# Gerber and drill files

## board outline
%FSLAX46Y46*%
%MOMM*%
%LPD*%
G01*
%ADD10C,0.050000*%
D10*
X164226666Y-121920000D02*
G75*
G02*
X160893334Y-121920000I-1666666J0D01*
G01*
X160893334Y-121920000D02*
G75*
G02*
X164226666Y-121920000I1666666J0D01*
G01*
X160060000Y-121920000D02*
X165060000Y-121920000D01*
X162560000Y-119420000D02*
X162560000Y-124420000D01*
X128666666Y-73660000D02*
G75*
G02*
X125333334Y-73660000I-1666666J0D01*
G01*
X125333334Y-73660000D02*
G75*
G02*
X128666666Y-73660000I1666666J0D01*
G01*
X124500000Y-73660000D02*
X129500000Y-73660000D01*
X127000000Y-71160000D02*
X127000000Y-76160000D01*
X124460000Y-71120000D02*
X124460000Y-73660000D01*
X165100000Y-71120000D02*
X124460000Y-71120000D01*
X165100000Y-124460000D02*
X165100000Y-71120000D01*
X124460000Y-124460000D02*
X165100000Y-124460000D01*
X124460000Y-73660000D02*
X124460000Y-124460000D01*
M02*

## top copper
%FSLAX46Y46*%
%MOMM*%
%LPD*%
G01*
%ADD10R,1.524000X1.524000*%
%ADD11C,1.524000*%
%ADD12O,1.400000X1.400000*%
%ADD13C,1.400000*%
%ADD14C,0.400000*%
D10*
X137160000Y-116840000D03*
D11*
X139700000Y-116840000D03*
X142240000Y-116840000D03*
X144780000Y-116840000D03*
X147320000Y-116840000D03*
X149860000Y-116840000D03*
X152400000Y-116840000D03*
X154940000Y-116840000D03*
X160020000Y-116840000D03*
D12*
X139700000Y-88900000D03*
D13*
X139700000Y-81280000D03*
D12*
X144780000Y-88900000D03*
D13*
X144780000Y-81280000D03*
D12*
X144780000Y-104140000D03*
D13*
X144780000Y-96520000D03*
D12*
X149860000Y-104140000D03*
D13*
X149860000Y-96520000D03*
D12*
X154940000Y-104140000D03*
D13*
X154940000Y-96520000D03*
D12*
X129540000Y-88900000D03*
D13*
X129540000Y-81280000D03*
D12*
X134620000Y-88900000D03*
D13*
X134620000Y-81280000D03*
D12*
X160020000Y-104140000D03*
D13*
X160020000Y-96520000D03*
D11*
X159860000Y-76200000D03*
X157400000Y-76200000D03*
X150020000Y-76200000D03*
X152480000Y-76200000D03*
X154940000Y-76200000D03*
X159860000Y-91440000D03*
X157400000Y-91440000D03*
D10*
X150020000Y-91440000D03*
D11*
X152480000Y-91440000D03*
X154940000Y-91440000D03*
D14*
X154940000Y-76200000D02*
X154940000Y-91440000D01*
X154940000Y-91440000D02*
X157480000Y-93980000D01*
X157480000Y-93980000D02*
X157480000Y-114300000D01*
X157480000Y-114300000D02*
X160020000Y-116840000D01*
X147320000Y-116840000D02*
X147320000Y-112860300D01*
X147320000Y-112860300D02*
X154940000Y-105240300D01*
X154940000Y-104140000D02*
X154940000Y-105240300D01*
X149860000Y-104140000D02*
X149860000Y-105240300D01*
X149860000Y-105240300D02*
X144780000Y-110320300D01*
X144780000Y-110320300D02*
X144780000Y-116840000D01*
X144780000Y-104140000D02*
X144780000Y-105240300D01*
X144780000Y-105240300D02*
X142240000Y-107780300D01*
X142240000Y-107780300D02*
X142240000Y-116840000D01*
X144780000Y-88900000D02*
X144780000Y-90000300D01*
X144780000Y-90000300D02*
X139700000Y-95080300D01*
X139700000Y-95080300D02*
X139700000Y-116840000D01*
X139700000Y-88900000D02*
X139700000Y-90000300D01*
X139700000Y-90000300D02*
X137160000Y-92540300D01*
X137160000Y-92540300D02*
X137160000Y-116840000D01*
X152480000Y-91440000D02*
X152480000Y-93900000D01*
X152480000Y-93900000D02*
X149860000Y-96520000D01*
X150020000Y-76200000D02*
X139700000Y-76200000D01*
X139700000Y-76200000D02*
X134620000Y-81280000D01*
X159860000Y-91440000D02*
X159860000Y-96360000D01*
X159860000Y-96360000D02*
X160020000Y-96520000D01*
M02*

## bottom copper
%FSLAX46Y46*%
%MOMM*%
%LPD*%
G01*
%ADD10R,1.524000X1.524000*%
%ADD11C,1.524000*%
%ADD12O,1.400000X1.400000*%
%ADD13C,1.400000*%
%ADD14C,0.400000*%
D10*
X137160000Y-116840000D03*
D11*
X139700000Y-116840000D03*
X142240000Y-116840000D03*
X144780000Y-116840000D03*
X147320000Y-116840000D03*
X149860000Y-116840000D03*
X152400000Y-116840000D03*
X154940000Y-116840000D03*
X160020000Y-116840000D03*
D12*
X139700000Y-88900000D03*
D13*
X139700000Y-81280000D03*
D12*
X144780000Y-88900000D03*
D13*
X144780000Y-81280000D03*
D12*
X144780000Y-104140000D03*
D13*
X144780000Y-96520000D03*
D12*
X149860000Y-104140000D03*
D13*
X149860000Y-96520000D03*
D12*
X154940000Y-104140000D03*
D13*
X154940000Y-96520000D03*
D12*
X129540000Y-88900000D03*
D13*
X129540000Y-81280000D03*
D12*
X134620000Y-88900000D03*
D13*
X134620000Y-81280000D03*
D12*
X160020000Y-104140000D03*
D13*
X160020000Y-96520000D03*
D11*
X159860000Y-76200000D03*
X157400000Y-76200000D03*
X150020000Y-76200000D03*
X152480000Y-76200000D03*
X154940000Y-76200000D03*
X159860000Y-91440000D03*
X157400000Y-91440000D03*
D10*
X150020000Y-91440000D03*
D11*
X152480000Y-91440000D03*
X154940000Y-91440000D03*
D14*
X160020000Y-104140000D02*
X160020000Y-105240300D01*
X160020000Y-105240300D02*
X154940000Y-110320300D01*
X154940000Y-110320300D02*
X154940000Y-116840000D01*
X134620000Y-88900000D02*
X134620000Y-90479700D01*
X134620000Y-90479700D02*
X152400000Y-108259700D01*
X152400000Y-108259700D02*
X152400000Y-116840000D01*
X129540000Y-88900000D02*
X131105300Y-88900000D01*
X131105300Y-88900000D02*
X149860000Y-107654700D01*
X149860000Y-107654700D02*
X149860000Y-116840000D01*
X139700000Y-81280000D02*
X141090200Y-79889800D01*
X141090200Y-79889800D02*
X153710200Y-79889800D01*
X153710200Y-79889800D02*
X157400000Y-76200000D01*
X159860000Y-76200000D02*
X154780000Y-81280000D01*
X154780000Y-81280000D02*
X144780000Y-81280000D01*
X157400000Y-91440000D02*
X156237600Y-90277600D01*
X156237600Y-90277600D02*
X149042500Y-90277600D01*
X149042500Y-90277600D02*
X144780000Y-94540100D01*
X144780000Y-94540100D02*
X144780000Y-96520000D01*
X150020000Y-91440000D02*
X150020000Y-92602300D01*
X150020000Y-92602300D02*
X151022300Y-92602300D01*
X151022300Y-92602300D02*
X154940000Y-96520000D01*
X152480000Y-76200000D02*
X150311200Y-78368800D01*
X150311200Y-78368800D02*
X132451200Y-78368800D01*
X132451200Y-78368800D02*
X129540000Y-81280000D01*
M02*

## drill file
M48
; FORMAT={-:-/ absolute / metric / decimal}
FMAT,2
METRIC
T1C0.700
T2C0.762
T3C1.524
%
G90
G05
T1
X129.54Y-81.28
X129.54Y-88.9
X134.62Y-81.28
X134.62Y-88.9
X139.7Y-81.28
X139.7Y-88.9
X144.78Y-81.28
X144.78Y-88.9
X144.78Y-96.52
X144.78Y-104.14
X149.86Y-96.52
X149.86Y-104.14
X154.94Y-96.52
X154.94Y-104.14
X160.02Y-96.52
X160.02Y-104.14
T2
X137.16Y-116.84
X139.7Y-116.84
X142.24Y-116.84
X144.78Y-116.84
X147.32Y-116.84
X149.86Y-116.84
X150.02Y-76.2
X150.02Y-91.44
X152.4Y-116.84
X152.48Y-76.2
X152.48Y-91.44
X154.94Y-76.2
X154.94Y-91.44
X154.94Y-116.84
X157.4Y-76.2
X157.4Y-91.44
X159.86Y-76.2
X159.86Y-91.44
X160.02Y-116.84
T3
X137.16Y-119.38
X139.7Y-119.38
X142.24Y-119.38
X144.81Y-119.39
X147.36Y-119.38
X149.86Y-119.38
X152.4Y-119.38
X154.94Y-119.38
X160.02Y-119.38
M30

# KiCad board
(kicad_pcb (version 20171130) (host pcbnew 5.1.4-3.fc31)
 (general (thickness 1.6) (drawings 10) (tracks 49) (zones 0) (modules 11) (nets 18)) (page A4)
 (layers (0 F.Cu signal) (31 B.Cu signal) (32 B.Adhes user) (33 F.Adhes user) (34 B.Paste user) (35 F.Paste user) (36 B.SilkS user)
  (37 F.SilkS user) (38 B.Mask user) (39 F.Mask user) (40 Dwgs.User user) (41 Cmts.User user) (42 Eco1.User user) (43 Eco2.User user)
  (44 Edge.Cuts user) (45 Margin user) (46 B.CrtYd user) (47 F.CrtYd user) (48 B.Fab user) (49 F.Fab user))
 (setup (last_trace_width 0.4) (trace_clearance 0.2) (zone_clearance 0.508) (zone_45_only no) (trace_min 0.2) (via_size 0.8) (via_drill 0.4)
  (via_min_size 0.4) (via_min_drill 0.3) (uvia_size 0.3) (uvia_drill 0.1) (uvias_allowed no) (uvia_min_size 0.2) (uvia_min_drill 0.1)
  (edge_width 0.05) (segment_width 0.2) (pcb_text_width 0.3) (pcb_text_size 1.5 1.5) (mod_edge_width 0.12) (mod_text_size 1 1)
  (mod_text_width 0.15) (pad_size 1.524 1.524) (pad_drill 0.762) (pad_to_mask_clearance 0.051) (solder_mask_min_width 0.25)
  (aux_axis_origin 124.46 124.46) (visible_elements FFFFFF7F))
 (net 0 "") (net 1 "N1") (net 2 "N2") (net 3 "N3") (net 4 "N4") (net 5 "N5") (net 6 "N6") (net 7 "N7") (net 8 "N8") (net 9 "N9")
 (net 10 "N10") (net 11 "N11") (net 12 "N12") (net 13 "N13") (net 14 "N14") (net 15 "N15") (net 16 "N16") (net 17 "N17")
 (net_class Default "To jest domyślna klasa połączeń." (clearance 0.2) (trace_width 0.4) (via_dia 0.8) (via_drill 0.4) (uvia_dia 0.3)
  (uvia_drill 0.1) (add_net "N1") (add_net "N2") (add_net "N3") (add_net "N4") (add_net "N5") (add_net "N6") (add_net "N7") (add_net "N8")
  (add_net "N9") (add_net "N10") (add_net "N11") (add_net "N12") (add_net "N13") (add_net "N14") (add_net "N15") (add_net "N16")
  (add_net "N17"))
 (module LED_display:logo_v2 (layer F.Cu) (at 129.54 114.3 90)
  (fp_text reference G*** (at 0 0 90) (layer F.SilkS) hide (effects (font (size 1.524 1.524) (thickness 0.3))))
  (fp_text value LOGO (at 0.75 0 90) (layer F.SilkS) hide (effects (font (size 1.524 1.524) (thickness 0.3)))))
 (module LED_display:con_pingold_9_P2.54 (layer F.Cu) (at 137.16 116.84)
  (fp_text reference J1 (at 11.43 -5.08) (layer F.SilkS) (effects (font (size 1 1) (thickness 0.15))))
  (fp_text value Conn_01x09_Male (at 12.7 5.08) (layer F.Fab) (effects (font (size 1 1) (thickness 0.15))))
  (pad 1 thru_hole rect (at 0 0) (size 1.524 1.524) (drill 0.762) (layers *.Cu *.Mask) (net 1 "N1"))
  (pad 2 thru_hole circle (at 2.54 0) (size 1.524 1.524) (drill 0.762) (layers *.Cu *.Mask) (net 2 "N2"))
  (pad 3 thru_hole circle (at 5.08 0) (size 1.524 1.524) (drill 0.762) (layers *.Cu *.Mask) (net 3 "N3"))
  (pad 4 thru_hole circle (at 7.62 0) (size 1.524 1.524) (drill 0.762) (layers *.Cu *.Mask) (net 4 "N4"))
  (pad 5 thru_hole circle (at 10.16 0) (size 1.524 1.524) (drill 0.762) (layers *.Cu *.Mask) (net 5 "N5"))
  (pad 6 thru_hole circle (at 12.7 0) (size 1.524 1.524) (drill 0.762) (layers *.Cu *.Mask) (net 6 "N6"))
  (pad 7 thru_hole circle (at 15.24 0) (size 1.524 1.524) (drill 0.762) (layers *.Cu *.Mask) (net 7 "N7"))
  (pad 8 thru_hole circle (at 17.78 0) (size 1.524 1.524) (drill 0.762) (layers *.Cu *.Mask) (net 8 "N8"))
  (pad 9 thru_hole circle (at 22.86 0) (size 1.524 1.524) (drill 0.762) (layers *.Cu *.Mask) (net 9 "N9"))
  (pad "" np_thru_hole circle (at 0 2.54) (size 1.524 1.524) (drill 1.524) (layers *.Cu *.Mask))
  (pad "" np_thru_hole circle (at 2.54 2.54) (size 1.524 1.524) (drill 1.524) (layers *.Cu *.Mask))
  (pad "" np_thru_hole circle (at 5.08 2.54) (size 1.524 1.524) (drill 1.524) (layers *.Cu *.Mask))
  (pad "" np_thru_hole circle (at 7.65 2.55) (size 1.524 1.524) (drill 1.524) (layers *.Cu *.Mask))
  (pad "" np_thru_hole circle (at 10.2 2.54) (size 1.524 1.524) (drill 1.524) (layers *.Cu *.Mask))
  (pad "" np_thru_hole circle (at 12.7 2.54) (size 1.524 1.524) (drill 1.524) (layers *.Cu *.Mask))
  (pad "" np_thru_hole circle (at 15.24 2.54) (size 1.524 1.524) (drill 1.524) (layers *.Cu *.Mask))
  (pad "" np_thru_hole circle (at 17.78 2.54) (size 1.524 1.524) (drill 1.524) (layers *.Cu *.Mask))
  (pad "" np_thru_hole circle (at 22.86 2.54) (size 1.524 1.524) (drill 1.524) (layers *.Cu *.Mask)))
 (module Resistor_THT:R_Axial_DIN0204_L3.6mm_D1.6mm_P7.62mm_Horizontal (layer F.Cu) (at 139.7 81.28 270)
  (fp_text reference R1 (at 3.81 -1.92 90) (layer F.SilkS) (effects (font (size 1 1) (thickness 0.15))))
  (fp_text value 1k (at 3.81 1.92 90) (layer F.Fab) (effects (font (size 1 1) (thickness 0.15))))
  (pad 2 thru_hole oval (at 7.62 0 270) (size 1.4 1.4) (drill 0.7) (layers *.Cu *.Mask) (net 1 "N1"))
  (pad 1 thru_hole circle (at 0 0 270) (size 1.4 1.4) (drill 0.7) (layers *.Cu *.Mask) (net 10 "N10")))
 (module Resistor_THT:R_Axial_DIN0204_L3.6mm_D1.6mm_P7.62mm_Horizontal (layer F.Cu) (at 144.78 81.28 270)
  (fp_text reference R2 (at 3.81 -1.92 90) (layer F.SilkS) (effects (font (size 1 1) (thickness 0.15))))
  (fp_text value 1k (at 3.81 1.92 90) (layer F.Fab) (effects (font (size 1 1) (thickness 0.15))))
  (pad 2 thru_hole oval (at 7.62 0 270) (size 1.4 1.4) (drill 0.7) (layers *.Cu *.Mask) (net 2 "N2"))
  (pad 1 thru_hole circle (at 0 0 270) (size 1.4 1.4) (drill 0.7) (layers *.Cu *.Mask) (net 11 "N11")))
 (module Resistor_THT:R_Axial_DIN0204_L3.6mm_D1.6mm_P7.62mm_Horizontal (layer F.Cu) (at 144.78 96.52 270)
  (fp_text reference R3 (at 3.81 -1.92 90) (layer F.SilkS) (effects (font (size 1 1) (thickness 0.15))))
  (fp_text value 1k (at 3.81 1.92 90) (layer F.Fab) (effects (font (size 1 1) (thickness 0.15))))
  (pad 2 thru_hole oval (at 7.62 0 270) (size 1.4 1.4) (drill 0.7) (layers *.Cu *.Mask) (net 3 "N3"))
  (pad 1 thru_hole circle (at 0 0 270) (size 1.4 1.4) (drill 0.7) (layers *.Cu *.Mask) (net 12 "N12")))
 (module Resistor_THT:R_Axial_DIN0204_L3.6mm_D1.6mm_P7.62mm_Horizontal (layer F.Cu) (at 149.86 96.52 270)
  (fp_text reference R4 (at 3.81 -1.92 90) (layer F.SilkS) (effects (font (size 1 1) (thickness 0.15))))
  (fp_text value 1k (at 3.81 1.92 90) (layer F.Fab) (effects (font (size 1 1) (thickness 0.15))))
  (pad 2 thru_hole oval (at 7.62 0 270) (size 1.4 1.4) (drill 0.7) (layers *.Cu *.Mask) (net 4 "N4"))
  (pad 1 thru_hole circle (at 0 0 270) (size 1.4 1.4) (drill 0.7) (layers *.Cu *.Mask) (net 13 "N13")))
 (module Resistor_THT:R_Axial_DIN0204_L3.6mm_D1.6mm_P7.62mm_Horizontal (layer F.Cu) (at 154.94 96.52 270)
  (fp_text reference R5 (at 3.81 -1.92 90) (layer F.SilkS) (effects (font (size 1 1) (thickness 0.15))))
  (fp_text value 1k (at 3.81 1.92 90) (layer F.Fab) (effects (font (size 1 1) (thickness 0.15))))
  (pad 2 thru_hole oval (at 7.62 0 270) (size 1.4 1.4) (drill 0.7) (layers *.Cu *.Mask) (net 5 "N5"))
  (pad 1 thru_hole circle (at 0 0 270) (size 1.4 1.4) (drill 0.7) (layers *.Cu *.Mask) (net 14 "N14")))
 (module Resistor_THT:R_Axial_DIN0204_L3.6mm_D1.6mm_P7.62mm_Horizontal (layer F.Cu) (at 129.54 81.28 270)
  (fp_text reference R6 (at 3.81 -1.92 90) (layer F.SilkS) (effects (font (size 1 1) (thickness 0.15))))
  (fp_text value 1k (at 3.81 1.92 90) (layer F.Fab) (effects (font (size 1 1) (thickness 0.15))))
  (pad 2 thru_hole oval (at 7.62 0 270) (size 1.4 1.4) (drill 0.7) (layers *.Cu *.Mask) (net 6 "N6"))
  (pad 1 thru_hole circle (at 0 0 270) (size 1.4 1.4) (drill 0.7) (layers *.Cu *.Mask) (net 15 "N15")))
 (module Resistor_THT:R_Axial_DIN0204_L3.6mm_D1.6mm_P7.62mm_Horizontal (layer F.Cu) (at 134.62 81.28 270)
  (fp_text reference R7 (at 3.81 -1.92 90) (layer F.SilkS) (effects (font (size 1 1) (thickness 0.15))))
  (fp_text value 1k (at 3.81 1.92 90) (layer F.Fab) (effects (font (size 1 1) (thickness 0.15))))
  (pad 2 thru_hole oval (at 7.62 0 270) (size 1.4 1.4) (drill 0.7) (layers *.Cu *.Mask) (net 7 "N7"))
  (pad 1 thru_hole circle (at 0 0 270) (size 1.4 1.4) (drill 0.7) (layers *.Cu *.Mask) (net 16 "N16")))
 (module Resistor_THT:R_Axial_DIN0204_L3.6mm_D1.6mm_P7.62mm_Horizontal (layer F.Cu) (at 160.02 96.52 270)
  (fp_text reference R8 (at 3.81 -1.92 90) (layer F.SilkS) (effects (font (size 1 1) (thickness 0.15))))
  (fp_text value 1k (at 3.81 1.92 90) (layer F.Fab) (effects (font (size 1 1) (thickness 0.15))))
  (pad 2 thru_hole oval (at 7.62 0 270) (size 1.4 1.4) (drill 0.7) (layers *.Cu *.Mask) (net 8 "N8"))
  (pad 1 thru_hole circle (at 0 0 270) (size 1.4 1.4) (drill 0.7) (layers *.Cu *.Mask) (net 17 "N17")))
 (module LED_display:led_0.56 (layer F.Cu) (at 154.94 83.82)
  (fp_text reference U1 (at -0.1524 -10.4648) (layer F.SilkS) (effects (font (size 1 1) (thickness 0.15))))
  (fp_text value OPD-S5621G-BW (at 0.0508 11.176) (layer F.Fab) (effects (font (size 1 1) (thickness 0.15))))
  (pad 6 thru_hole circle (at 4.92 -7.62) (size 1.524 1.524) (drill 0.762) (layers *.Cu *.Mask) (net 11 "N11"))
  (pad 7 thru_hole circle (at 2.46 -7.62) (size 1.524 1.524) (drill 0.762) (layers *.Cu *.Mask) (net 10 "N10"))
  (pad 10 thru_hole circle (at -4.92 -7.62) (size 1.524 1.524) (drill 0.762) (layers *.Cu *.Mask) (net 16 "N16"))
  (pad 9 thru_hole circle (at -2.46 -7.62) (size 1.524 1.524) (drill 0.762) (layers *.Cu *.Mask) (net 15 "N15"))
  (pad 8 thru_hole circle (at 0 -7.62) (size 1.524 1.524) (drill 0.762) (layers *.Cu *.Mask) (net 9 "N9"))
  (pad 5 thru_hole circle (at 4.92 7.62) (size 1.524 1.524) (drill 0.762) (layers *.Cu *.Mask) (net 17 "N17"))
  (pad 4 thru_hole circle (at 2.46 7.62) (size 1.524 1.524) (drill 0.762) (layers *.Cu *.Mask) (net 12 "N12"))
  (pad 1 thru_hole rect (at -4.92 7.62) (size 1.524 1.524) (drill 0.762) (layers *.Cu *.Mask) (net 14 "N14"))
  (pad 2 thru_hole circle (at -2.46 7.62) (size 1.524 1.524) (drill 0.762) (layers *.Cu *.Mask) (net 13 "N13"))
  (pad 3 thru_hole circle (at 0 7.62) (size 1.524 1.524) (drill 0.762) (layers *.Cu *.Mask) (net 9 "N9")))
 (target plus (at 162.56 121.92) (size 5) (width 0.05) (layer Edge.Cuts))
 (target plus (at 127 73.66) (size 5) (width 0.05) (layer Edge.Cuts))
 (gr_line (start 124.46 71.12) (end 124.46 73.66) (layer Edge.Cuts) (width 0.05))
 (gr_line (start 165.1 71.12) (end 124.46 71.12) (layer Edge.Cuts) (width 0.05))
 (gr_line (start 165.1 124.46) (end 165.1 71.12) (layer Edge.Cuts) (width 0.05))
 (gr_line (start 124.46 124.46) (end 165.1 124.46) (layer Edge.Cuts) (width 0.05))
 (gr_line (start 124.46 73.66) (end 124.46 124.46) (layer Edge.Cuts) (width 0.05))
 (segment (start 154.94 76.2) (end 154.94 91.44) (width 0.4) (layer F.Cu) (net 9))
 (segment (start 154.94 91.44) (end 157.48 93.98) (width 0.4) (layer F.Cu) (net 9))
 (segment (start 157.48 93.98) (end 157.48 114.3) (width 0.4) (layer F.Cu) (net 9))
 (segment (start 157.48 114.3) (end 160.02 116.84) (width 0.4) (layer F.Cu) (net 9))
 (segment (start 160.02 104.14) (end 160.02 105.2403) (width 0.4) (layer B.Cu) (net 8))
 (segment (start 160.02 105.2403) (end 154.94 110.3203) (width 0.4) (layer B.Cu) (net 8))
 (segment (start 154.94 110.3203) (end 154.94 116.84) (width 0.4) (layer B.Cu) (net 8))
 (segment (start 134.62 88.9) (end 134.62 90.4797) (width 0.4) (layer B.Cu) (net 7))
 (segment (start 134.62 90.4797) (end 152.4 108.2597) (width 0.4) (layer B.Cu) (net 7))
 (segment (start 152.4 108.2597) (end 152.4 116.84) (width 0.4) (layer B.Cu) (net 7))
 (segment (start 129.54 88.9) (end 131.1053 88.9) (width 0.4) (layer B.Cu) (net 6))
 (segment (start 131.1053 88.9) (end 149.86 107.6547) (width 0.4) (layer B.Cu) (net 6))
 (segment (start 149.86 107.6547) (end 149.86 116.84) (width 0.4) (layer B.Cu) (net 6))
 (segment (start 147.32 116.84) (end 147.32 112.8603) (width 0.4) (layer F.Cu) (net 5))
 (segment (start 147.32 112.8603) (end 154.94 105.2403) (width 0.4) (layer F.Cu) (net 5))
 (segment (start 154.94 104.14) (end 154.94 105.2403) (width 0.4) (layer F.Cu) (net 5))
 (segment (start 149.86 104.14) (end 149.86 105.2403) (width 0.4) (layer F.Cu) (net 4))
 (segment (start 149.86 105.2403) (end 144.78 110.3203) (width 0.4) (layer F.Cu) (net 4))
 (segment (start 144.78 110.3203) (end 144.78 116.84) (width 0.4) (layer F.Cu) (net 4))
 (segment (start 144.78 104.14) (end 144.78 105.2403) (width 0.4) (layer F.Cu) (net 3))
 (segment (start 144.78 105.2403) (end 142.24 107.7803) (width 0.4) (layer F.Cu) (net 3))
 (segment (start 142.24 107.7803) (end 142.24 116.84) (width 0.4) (layer F.Cu) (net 3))
 (segment (start 144.78 88.9) (end 144.78 90.0003) (width 0.4) (layer F.Cu) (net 2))
 (segment (start 144.78 90.0003) (end 139.7 95.0803) (width 0.4) (layer F.Cu) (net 2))
 (segment (start 139.7 95.0803) (end 139.7 116.84) (width 0.4) (layer F.Cu) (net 2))
 (segment (start 139.7 88.9) (end 139.7 90.0003) (width 0.4) (layer F.Cu) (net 1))
 (segment (start 139.7 90.0003) (end 137.16 92.5403) (width 0.4) (layer F.Cu) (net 1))
 (segment (start 137.16 92.5403) (end 137.16 116.84) (width 0.4) (layer F.Cu) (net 1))
 (segment (start 139.7 81.28) (end 141.0902 79.8898) (width 0.4) (layer B.Cu) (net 10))
 (segment (start 141.0902 79.8898) (end 153.7102 79.8898) (width 0.4) (layer B.Cu) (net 10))
 (segment (start 153.7102 79.8898) (end 157.4 76.2) (width 0.4) (layer B.Cu) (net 10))
 (segment (start 159.86 76.2) (end 154.78 81.28) (width 0.4) (layer B.Cu) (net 11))
 (segment (start 154.78 81.28) (end 144.78 81.28) (width 0.4) (layer B.Cu) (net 11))
 (segment (start 157.4 91.44) (end 156.2376 90.2776) (width 0.4) (layer B.Cu) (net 12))
 (segment (start 156.2376 90.2776) (end 149.0425 90.2776) (width 0.4) (layer B.Cu) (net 12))
 (segment (start 149.0425 90.2776) (end 144.78 94.5401) (width 0.4) (layer B.Cu) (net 12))
 (segment (start 144.78 94.5401) (end 144.78 96.52) (width 0.4) (layer B.Cu) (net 12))
 (segment (start 152.48 91.44) (end 152.48 93.9) (width 0.4) (layer F.Cu) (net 13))
 (segment (start 152.48 93.9) (end 149.86 96.52) (width 0.4) (layer F.Cu) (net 13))
 (segment (start 150.02 91.44) (end 150.02 92.6023) (width 0.4) (layer B.Cu) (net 14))
 (segment (start 150.02 92.6023) (end 151.0223 92.6023) (width 0.4) (layer B.Cu) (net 14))
 (segment (start 151.0223 92.6023) (end 154.94 96.52) (width 0.4) (layer B.Cu) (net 14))
 (segment (start 152.48 76.2) (end 150.3112 78.3688) (width 0.4) (layer B.Cu) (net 15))
 (segment (start 150.3112 78.3688) (end 132.4512 78.3688) (width 0.4) (layer B.Cu) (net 15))
 (segment (start 132.4512 78.3688) (end 129.54 81.28) (width 0.4) (layer B.Cu) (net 15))
 (segment (start 150.02 76.2) (end 139.7 76.2) (width 0.4) (layer F.Cu) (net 16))
 (segment (start 139.7 76.2) (end 134.62 81.28) (width 0.4) (layer F.Cu) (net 16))
 (segment (start 159.86 91.44) (end 159.86 96.36) (width 0.4) (layer F.Cu) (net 17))
 (segment (start 159.86 96.36) (end 160.02 96.52) (width 0.4) (layer F.Cu) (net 17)))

